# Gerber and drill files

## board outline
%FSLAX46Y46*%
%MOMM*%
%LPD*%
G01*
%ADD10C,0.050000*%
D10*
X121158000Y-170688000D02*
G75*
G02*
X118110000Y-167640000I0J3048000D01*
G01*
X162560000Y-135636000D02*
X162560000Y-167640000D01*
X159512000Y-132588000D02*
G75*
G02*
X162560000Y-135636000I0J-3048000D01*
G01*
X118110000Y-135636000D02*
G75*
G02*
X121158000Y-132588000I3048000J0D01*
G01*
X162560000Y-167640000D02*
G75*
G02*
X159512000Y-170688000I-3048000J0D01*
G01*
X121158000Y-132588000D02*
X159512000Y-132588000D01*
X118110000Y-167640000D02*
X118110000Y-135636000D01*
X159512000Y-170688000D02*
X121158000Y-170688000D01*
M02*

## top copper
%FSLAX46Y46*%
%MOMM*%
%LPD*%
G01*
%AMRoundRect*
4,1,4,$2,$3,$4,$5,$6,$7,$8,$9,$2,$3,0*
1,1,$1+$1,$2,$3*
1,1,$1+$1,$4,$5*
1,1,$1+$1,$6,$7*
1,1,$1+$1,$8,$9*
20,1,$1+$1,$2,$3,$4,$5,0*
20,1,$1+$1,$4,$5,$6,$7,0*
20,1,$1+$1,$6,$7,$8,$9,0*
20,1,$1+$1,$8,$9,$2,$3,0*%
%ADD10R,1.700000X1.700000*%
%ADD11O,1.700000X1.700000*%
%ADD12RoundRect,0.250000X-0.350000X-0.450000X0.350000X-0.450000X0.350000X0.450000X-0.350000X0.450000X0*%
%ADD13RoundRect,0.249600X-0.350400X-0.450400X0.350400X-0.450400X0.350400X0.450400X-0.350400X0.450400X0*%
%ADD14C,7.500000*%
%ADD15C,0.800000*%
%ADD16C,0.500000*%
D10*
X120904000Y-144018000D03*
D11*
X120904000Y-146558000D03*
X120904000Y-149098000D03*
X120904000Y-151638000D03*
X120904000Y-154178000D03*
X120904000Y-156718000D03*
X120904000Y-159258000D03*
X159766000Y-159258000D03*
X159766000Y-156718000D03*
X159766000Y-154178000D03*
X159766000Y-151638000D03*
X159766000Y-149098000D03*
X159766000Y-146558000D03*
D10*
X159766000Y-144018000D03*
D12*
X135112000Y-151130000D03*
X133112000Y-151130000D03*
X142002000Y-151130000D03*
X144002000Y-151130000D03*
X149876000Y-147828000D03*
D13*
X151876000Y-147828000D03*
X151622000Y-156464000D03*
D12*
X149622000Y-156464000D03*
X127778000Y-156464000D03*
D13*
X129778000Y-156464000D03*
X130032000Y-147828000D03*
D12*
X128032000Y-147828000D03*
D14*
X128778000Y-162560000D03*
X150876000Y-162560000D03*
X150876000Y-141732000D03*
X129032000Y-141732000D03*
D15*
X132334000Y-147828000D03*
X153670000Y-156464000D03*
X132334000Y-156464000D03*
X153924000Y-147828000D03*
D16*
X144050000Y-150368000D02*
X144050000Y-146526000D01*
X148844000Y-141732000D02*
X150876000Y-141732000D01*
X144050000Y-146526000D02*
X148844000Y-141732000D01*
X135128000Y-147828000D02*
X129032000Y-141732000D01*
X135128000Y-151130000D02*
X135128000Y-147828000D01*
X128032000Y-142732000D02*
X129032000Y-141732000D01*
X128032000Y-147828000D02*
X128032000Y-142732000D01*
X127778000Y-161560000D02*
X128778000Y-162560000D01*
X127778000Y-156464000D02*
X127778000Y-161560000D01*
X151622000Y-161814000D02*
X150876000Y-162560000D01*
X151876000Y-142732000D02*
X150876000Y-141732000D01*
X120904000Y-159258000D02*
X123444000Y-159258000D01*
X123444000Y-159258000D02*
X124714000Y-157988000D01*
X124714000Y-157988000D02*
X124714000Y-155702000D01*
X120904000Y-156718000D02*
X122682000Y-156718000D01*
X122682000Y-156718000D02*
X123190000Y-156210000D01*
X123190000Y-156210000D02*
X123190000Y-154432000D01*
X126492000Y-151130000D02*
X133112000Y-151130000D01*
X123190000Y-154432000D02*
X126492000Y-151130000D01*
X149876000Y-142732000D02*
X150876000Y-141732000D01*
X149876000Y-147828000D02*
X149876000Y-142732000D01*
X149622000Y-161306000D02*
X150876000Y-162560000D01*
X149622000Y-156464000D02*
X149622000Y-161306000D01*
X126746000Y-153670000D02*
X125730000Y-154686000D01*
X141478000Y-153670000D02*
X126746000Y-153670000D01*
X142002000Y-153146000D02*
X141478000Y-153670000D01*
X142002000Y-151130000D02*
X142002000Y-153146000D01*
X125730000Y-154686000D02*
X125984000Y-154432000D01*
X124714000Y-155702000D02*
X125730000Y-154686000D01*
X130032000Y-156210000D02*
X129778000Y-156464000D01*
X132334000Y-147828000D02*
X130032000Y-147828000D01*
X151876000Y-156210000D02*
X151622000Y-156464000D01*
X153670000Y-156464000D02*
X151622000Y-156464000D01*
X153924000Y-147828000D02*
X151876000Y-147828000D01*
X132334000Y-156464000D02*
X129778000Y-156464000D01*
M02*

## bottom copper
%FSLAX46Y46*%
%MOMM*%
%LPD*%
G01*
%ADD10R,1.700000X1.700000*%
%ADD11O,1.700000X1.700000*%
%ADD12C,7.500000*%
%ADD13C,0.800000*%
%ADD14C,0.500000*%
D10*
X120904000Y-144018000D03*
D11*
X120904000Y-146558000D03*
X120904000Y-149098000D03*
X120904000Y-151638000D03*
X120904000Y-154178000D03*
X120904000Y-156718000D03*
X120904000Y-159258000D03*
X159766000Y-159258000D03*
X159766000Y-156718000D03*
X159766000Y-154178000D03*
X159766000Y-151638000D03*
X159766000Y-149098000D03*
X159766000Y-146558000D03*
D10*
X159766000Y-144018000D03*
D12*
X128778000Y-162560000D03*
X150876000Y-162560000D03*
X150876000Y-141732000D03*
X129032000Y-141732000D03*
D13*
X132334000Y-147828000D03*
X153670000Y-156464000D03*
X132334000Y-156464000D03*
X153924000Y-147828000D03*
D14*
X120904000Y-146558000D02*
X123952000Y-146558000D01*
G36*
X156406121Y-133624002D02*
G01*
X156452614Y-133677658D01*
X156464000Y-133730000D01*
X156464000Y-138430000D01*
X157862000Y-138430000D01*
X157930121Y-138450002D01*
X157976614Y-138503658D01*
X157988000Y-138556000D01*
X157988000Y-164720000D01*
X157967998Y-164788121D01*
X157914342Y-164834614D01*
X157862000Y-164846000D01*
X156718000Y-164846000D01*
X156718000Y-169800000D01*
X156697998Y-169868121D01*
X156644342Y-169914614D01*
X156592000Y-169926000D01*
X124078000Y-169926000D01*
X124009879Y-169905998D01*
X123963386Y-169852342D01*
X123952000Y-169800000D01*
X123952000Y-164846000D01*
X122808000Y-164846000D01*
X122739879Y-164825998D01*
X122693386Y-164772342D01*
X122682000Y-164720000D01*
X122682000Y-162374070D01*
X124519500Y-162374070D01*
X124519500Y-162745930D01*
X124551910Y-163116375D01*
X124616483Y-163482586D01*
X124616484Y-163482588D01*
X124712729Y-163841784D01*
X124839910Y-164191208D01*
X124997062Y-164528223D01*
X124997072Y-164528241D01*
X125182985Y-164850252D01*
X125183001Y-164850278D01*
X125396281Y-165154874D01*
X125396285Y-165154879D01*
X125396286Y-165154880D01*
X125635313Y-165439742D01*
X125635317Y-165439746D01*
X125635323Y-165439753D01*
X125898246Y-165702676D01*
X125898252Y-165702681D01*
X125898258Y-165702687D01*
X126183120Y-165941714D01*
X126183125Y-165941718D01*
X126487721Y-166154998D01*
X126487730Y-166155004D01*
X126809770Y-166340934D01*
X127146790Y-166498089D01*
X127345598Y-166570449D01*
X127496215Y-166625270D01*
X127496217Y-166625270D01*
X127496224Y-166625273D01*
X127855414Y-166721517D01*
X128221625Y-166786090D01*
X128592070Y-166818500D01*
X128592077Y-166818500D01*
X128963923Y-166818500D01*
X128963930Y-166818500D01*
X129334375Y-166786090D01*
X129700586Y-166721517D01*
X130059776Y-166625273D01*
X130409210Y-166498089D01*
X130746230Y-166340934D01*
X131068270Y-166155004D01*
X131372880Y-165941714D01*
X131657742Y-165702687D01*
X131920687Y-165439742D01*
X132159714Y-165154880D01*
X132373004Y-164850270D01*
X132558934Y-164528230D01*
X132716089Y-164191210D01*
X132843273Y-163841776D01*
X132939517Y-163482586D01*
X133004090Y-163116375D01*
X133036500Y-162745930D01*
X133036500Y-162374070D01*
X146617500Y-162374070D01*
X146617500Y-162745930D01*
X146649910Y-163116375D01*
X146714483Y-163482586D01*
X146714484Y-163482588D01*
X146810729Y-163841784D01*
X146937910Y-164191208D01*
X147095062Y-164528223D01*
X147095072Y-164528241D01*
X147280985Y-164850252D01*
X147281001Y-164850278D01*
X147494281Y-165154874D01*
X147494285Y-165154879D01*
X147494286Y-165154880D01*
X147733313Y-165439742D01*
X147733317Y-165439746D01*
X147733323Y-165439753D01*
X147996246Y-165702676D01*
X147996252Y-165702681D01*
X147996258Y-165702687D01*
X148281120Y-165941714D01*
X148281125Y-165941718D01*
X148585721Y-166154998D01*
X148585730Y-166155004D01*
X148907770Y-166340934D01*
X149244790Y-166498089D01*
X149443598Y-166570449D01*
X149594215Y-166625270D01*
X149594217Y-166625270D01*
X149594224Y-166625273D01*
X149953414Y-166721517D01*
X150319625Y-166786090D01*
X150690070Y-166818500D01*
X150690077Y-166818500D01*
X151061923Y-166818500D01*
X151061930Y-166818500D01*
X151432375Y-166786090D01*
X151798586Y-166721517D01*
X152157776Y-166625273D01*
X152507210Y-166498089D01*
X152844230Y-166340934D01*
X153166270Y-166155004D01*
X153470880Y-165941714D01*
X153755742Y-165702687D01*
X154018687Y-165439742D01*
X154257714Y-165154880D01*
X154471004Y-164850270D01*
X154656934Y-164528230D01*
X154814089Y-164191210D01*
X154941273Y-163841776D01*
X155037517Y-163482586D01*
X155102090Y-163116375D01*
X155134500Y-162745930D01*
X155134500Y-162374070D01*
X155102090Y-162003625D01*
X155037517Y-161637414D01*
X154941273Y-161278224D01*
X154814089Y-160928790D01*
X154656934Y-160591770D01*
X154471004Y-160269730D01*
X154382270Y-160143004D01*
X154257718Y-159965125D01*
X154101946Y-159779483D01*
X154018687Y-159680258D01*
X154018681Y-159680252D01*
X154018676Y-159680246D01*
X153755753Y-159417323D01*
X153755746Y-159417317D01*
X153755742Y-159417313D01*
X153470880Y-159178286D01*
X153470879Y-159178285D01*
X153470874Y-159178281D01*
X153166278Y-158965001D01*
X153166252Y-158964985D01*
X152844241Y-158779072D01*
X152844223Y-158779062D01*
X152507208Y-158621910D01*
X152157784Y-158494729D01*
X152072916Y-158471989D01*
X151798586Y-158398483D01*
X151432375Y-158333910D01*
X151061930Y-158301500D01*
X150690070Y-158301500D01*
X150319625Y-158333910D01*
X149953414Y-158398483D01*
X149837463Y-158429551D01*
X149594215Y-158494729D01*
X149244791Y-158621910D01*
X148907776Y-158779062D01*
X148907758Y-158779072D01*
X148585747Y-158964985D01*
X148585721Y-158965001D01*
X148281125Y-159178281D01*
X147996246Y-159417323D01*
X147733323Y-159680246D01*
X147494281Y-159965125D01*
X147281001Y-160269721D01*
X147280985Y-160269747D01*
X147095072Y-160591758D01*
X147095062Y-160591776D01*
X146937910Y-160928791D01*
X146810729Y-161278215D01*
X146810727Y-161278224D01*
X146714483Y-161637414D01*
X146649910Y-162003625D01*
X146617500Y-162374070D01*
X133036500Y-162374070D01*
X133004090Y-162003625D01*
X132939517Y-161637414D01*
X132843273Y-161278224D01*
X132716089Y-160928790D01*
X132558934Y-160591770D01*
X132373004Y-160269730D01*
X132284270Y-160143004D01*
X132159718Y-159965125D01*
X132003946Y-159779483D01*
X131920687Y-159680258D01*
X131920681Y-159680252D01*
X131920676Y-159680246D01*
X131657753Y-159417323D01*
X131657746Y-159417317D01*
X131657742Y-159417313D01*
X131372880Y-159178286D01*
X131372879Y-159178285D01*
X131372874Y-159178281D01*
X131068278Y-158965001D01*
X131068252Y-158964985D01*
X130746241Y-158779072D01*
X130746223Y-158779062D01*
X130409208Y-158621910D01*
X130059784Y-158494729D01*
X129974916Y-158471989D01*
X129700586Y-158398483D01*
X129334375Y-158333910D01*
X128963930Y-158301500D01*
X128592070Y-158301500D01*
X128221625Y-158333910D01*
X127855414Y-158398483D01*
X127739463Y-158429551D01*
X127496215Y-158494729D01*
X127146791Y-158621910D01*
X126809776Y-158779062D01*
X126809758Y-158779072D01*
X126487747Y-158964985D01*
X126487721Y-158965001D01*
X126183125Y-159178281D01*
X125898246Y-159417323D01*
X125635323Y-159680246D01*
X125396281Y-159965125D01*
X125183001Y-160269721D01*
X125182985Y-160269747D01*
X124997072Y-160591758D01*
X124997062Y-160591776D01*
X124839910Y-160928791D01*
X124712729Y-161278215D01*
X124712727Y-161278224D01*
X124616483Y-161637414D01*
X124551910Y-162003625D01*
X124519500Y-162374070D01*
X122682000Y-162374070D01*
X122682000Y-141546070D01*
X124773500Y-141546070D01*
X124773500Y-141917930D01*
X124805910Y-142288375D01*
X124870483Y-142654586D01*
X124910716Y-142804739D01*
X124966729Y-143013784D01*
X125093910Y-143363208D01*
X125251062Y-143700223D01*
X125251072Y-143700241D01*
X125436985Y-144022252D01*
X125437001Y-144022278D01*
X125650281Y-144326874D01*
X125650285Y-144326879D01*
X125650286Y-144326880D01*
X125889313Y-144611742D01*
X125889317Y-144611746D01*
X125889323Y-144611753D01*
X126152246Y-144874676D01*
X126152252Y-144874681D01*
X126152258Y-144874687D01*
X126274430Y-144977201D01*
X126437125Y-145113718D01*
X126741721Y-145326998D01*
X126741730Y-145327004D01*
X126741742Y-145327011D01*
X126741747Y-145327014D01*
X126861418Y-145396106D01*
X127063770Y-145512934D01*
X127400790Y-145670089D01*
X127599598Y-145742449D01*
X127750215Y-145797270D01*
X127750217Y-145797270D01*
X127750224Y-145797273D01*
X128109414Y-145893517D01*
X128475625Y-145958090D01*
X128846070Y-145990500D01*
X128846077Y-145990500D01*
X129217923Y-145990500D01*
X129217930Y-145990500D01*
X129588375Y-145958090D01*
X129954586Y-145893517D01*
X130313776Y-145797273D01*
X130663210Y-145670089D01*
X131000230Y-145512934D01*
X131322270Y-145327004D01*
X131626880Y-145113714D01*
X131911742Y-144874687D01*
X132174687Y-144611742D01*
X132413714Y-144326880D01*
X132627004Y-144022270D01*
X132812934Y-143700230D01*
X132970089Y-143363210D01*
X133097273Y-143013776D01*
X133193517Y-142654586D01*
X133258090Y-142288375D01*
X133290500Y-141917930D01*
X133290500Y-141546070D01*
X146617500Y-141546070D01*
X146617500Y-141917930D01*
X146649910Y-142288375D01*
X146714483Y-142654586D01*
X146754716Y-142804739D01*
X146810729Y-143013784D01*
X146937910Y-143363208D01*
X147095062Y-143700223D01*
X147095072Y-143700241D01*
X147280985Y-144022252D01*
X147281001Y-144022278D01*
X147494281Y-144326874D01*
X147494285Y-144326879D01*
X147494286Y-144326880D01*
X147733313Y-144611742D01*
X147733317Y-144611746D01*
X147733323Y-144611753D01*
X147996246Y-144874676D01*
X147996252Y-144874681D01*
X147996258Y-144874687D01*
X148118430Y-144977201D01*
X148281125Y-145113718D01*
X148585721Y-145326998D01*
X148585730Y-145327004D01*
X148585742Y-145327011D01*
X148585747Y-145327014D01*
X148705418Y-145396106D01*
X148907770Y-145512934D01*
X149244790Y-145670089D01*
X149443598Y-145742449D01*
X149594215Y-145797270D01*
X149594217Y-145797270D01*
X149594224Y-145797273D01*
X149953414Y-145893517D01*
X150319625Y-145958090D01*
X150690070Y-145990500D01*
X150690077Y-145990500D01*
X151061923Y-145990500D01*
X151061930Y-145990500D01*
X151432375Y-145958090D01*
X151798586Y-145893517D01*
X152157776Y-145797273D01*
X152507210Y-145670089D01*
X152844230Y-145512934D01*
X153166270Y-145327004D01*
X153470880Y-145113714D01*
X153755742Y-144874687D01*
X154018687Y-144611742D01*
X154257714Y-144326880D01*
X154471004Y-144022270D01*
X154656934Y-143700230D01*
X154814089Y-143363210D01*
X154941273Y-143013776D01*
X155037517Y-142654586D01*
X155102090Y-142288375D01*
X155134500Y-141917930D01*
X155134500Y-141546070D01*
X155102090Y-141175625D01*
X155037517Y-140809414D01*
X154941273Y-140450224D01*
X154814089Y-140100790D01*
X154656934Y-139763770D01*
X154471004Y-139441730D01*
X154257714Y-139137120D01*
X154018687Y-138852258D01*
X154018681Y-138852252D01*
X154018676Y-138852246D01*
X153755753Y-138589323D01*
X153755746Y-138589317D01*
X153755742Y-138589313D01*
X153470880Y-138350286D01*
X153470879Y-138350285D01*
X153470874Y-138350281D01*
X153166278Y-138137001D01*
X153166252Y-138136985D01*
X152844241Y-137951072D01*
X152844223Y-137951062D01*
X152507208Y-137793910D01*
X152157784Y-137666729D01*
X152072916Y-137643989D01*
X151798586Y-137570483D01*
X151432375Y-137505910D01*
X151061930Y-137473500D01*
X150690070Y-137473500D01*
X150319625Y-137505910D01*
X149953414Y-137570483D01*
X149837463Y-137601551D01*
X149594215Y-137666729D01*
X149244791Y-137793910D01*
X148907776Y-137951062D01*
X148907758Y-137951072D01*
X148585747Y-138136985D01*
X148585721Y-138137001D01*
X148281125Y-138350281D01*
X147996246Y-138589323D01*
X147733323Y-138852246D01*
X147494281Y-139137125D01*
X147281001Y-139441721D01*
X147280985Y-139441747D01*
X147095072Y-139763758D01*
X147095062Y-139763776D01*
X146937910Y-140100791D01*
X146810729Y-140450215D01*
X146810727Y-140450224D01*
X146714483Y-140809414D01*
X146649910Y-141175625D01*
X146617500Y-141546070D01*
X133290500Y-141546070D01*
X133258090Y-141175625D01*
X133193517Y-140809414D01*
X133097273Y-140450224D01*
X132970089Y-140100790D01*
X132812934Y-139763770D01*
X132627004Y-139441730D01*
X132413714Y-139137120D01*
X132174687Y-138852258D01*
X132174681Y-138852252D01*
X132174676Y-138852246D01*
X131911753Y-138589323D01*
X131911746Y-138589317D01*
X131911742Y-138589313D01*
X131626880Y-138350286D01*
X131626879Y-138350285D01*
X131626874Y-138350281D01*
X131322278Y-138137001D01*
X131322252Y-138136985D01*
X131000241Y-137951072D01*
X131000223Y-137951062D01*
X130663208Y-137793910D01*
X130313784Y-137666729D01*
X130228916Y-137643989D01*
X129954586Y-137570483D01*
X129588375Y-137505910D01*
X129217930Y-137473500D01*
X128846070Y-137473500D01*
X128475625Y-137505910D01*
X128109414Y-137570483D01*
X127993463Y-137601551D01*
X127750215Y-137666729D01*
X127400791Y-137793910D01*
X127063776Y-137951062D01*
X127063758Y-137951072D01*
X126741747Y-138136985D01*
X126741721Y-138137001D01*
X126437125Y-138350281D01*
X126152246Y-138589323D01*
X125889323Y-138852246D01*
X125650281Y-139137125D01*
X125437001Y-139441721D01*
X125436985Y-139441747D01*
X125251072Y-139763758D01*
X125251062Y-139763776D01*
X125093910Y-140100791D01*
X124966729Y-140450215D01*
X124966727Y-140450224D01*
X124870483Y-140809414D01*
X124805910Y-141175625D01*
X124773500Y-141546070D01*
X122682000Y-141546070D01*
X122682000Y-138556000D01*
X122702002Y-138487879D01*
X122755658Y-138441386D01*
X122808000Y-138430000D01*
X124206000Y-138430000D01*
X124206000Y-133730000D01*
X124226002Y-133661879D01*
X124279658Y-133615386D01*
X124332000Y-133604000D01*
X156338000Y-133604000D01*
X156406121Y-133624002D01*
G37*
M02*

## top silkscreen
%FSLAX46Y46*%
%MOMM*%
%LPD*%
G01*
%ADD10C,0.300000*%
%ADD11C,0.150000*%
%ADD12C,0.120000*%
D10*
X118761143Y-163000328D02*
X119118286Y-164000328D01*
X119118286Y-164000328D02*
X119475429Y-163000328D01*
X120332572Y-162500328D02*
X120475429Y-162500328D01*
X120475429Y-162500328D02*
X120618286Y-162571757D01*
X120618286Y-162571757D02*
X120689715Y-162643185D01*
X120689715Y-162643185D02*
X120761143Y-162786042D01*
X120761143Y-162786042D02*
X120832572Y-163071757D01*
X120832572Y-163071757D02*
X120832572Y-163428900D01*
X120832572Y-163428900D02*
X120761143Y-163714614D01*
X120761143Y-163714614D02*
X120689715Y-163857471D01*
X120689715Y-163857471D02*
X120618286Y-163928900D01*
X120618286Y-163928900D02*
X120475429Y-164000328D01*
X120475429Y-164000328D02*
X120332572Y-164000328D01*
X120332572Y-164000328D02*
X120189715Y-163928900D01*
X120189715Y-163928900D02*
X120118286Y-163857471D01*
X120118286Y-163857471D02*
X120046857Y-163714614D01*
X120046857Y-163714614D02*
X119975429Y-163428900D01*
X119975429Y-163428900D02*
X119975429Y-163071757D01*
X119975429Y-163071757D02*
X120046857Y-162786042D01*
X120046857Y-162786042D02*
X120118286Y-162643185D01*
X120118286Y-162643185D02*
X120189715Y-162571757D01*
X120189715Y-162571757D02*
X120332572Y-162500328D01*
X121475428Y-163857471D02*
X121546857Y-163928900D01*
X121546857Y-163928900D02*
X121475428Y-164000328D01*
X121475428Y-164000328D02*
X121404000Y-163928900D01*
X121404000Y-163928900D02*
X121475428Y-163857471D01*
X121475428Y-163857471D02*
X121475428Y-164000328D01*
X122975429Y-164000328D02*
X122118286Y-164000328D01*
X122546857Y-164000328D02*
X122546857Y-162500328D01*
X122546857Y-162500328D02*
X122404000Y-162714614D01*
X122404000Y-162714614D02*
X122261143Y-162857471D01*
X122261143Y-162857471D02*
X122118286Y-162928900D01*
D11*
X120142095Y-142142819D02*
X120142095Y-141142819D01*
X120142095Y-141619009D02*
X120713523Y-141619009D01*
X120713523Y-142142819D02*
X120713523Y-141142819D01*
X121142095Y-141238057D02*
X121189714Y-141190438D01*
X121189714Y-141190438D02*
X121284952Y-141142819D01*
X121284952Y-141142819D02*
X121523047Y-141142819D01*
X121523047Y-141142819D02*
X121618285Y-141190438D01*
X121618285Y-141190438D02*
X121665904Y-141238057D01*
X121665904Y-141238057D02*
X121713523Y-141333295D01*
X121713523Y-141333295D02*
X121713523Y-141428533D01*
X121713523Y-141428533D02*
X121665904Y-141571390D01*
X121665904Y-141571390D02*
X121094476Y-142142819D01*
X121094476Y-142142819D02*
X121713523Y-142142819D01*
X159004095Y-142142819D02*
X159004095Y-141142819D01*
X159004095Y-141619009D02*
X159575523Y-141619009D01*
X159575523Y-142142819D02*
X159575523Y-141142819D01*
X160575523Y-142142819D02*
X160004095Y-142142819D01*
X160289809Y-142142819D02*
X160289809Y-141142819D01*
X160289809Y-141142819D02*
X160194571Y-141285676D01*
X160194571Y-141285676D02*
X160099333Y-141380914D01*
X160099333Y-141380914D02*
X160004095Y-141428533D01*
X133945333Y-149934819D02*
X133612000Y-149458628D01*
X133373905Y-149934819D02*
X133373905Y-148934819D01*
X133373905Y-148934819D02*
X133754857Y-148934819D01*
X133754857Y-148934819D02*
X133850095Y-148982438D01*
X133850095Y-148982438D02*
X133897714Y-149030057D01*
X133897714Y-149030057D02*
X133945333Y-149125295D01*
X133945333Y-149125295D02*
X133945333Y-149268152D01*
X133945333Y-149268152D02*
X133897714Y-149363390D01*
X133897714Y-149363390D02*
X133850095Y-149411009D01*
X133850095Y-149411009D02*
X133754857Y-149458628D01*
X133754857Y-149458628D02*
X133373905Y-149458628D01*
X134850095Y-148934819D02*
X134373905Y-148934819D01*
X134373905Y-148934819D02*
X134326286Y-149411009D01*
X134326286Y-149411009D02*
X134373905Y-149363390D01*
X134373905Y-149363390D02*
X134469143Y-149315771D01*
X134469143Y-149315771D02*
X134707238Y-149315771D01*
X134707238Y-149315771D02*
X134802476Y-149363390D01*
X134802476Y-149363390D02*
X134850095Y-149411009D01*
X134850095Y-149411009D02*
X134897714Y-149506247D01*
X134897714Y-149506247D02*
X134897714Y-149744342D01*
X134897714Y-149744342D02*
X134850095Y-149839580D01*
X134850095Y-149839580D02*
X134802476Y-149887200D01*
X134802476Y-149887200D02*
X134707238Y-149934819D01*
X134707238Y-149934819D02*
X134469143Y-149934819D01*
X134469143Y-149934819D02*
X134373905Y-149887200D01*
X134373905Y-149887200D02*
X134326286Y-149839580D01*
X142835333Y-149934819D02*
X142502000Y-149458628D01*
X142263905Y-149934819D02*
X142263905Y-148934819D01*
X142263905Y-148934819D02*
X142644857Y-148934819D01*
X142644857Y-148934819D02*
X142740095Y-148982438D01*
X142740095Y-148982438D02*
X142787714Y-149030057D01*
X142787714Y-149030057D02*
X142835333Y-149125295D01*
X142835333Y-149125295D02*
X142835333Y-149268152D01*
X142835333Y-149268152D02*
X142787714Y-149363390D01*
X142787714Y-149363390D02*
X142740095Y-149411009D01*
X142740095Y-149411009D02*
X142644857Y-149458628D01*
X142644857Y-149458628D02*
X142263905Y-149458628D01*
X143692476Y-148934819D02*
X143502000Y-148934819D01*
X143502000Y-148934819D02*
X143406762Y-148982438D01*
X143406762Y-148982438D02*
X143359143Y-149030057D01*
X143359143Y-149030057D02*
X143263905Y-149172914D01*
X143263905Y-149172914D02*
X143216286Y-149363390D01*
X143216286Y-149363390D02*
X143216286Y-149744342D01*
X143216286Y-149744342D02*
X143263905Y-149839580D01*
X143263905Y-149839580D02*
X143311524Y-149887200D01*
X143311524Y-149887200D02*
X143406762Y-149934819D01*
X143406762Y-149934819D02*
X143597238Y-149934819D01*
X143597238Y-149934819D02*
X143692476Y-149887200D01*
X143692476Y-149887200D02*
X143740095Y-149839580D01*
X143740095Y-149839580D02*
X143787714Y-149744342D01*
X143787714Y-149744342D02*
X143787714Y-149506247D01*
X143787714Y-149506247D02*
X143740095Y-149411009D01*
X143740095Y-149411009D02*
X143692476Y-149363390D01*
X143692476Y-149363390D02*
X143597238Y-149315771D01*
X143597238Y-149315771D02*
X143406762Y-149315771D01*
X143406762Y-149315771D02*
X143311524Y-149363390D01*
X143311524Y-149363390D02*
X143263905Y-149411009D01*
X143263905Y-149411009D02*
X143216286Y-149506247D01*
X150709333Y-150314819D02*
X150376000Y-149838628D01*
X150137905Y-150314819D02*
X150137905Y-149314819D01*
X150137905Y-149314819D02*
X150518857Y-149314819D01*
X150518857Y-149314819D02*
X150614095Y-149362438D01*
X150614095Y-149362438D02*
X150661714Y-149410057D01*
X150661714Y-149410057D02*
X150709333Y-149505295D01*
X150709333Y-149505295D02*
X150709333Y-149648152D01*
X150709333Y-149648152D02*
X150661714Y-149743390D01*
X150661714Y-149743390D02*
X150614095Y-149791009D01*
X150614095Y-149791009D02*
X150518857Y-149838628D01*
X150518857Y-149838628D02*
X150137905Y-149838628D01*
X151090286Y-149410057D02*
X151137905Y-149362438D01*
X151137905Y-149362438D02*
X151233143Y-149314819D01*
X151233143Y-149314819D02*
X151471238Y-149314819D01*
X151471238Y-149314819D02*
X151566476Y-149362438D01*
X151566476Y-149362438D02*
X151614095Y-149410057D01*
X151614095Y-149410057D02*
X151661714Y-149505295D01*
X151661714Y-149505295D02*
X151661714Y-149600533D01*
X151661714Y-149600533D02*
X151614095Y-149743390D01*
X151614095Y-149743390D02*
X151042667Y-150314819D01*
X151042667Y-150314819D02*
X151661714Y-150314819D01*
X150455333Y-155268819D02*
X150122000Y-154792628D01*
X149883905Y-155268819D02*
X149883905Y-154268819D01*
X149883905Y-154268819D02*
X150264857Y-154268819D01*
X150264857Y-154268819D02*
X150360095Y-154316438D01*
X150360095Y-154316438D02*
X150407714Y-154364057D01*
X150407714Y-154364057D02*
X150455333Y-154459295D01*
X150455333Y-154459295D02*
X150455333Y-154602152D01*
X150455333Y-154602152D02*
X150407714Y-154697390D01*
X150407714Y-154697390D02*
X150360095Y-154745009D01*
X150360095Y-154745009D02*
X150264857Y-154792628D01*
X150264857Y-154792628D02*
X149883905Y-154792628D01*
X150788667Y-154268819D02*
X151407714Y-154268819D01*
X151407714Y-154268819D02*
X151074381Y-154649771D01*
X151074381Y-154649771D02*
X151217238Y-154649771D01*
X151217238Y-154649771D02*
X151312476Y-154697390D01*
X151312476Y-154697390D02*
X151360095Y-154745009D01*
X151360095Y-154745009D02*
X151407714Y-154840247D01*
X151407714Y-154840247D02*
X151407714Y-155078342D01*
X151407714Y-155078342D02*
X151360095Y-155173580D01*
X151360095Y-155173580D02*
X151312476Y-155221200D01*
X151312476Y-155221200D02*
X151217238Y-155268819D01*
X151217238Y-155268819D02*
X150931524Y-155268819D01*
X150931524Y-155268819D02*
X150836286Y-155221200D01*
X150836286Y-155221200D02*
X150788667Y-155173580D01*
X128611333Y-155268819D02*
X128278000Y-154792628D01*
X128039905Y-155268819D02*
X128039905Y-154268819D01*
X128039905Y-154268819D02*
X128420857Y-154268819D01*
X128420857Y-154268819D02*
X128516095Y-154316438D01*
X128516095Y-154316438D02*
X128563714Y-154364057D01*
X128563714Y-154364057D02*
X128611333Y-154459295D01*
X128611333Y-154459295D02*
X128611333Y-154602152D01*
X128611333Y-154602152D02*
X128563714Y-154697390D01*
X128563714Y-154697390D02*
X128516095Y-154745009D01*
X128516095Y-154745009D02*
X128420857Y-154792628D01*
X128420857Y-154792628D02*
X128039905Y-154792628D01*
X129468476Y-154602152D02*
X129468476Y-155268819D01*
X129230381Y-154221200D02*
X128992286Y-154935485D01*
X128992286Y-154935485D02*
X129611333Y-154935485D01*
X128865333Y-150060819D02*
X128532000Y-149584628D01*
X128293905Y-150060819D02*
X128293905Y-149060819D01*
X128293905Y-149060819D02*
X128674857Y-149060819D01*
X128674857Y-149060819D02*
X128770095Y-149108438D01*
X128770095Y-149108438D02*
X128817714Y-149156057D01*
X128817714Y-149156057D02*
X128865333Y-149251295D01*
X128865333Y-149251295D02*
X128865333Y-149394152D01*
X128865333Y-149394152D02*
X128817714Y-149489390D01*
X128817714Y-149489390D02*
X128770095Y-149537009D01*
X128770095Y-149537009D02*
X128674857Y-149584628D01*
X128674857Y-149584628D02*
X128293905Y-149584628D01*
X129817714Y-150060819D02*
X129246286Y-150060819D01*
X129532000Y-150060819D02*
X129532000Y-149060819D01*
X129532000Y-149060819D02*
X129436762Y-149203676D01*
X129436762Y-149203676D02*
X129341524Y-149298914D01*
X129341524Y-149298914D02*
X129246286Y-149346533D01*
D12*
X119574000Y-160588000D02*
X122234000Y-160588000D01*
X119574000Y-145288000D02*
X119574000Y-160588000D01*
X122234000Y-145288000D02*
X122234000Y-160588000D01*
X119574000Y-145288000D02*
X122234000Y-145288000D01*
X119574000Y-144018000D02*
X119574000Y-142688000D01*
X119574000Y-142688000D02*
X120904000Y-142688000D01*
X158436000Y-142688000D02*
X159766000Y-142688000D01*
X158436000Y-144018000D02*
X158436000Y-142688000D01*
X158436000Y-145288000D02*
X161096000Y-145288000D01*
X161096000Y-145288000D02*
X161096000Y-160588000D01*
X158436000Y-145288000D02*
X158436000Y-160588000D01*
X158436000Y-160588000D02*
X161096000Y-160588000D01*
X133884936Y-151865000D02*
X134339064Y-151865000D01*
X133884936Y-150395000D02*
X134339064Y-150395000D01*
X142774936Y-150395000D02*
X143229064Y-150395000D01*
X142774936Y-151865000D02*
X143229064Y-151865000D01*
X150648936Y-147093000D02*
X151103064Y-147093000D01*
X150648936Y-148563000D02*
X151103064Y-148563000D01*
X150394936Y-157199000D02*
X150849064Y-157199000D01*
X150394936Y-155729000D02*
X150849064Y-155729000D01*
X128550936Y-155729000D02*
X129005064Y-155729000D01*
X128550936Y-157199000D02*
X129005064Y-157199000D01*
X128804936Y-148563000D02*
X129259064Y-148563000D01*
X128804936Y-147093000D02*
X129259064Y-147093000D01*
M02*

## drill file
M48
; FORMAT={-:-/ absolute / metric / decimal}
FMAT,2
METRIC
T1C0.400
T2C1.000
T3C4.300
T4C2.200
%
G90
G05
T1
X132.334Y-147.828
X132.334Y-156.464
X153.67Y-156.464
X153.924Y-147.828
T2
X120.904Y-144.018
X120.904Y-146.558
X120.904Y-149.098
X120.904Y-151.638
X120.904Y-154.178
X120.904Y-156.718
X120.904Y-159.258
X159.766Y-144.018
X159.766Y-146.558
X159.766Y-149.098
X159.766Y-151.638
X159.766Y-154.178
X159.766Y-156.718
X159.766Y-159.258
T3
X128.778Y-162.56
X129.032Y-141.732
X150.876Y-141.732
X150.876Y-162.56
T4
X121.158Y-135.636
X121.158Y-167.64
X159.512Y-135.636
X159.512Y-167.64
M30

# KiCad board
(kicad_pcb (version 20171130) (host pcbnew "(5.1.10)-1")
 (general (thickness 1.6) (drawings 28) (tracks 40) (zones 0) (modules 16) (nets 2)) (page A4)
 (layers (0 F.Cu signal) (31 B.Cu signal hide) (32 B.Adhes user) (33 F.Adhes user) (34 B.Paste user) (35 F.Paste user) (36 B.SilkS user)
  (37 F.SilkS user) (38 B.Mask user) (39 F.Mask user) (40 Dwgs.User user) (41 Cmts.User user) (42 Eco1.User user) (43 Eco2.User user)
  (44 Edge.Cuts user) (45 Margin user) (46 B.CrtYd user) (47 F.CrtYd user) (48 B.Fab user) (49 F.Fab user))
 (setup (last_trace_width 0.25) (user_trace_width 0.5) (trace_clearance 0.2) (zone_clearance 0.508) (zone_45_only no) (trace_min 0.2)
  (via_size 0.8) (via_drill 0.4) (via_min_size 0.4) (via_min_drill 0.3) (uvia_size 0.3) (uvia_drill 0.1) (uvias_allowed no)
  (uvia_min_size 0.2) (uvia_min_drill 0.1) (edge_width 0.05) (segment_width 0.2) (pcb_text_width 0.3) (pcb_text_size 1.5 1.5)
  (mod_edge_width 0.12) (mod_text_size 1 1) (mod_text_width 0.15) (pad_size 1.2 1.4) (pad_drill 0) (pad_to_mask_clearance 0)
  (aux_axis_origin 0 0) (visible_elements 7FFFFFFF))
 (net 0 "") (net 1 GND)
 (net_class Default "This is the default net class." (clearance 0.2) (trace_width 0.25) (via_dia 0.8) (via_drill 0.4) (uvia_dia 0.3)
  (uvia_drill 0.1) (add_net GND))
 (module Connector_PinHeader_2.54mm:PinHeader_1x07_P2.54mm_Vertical (layer F.Cu) (at 120.904 144.018)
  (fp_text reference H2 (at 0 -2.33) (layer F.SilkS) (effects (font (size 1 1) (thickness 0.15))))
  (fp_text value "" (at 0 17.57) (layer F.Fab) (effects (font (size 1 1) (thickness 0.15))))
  (fp_line (start -1.33 16.57) (end 1.33 16.57) (layer F.SilkS) (width 0.12))
  (fp_line (start -1.33 1.27) (end -1.33 16.57) (layer F.SilkS) (width 0.12))
  (fp_line (start 1.33 1.27) (end 1.33 16.57) (layer F.SilkS) (width 0.12))
  (fp_line (start -1.33 1.27) (end 1.33 1.27) (layer F.SilkS) (width 0.12))
  (fp_line (start -1.33 0) (end -1.33 -1.33) (layer F.SilkS) (width 0.12))
  (fp_line (start -1.33 -1.33) (end 0 -1.33) (layer F.SilkS) (width 0.12))
  (pad 1 thru_hole rect (at 0 0) (size 1.7 1.7) (drill 1) (layers *.Cu *.Mask))
  (pad 2 thru_hole oval (at 0 2.54) (size 1.7 1.7) (drill 1) (layers *.Cu *.Mask) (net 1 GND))
  (pad 3 thru_hole oval (at 0 5.08) (size 1.7 1.7) (drill 1) (layers *.Cu *.Mask))
  (pad 4 thru_hole oval (at 0 7.62) (size 1.7 1.7) (drill 1) (layers *.Cu *.Mask))
  (pad 5 thru_hole oval (at 0 10.16) (size 1.7 1.7) (drill 1) (layers *.Cu *.Mask))
  (pad 6 thru_hole oval (at 0 12.7) (size 1.7 1.7) (drill 1) (layers *.Cu *.Mask))
  (pad 7 thru_hole oval (at 0 15.24) (size 1.7 1.7) (drill 1) (layers *.Cu *.Mask)))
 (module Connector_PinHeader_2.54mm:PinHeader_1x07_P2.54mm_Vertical (layer F.Cu) (at 159.766 144.018)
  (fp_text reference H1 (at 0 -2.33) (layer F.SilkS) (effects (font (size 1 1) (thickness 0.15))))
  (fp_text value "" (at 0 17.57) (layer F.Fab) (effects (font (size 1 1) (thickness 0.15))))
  (fp_line (start -1.33 -1.33) (end 0 -1.33) (layer F.SilkS) (width 0.12))
  (fp_line (start -1.33 0) (end -1.33 -1.33) (layer F.SilkS) (width 0.12))
  (fp_line (start -1.33 1.27) (end 1.33 1.27) (layer F.SilkS) (width 0.12))
  (fp_line (start 1.33 1.27) (end 1.33 16.57) (layer F.SilkS) (width 0.12))
  (fp_line (start -1.33 1.27) (end -1.33 16.57) (layer F.SilkS) (width 0.12))
  (fp_line (start -1.33 16.57) (end 1.33 16.57) (layer F.SilkS) (width 0.12))
  (pad 7 thru_hole oval (at 0 15.24) (size 1.7 1.7) (drill 1) (layers *.Cu *.Mask))
  (pad 6 thru_hole oval (at 0 12.7) (size 1.7 1.7) (drill 1) (layers *.Cu *.Mask))
  (pad 5 thru_hole oval (at 0 10.16) (size 1.7 1.7) (drill 1) (layers *.Cu *.Mask))
  (pad 4 thru_hole oval (at 0 7.62) (size 1.7 1.7) (drill 1) (layers *.Cu *.Mask))
  (pad 3 thru_hole oval (at 0 5.08) (size 1.7 1.7) (drill 1) (layers *.Cu *.Mask))
  (pad 2 thru_hole oval (at 0 2.54) (size 1.7 1.7) (drill 1) (layers *.Cu *.Mask))
  (pad 1 thru_hole rect (at 0 0) (size 1.7 1.7) (drill 1) (layers *.Cu *.Mask)))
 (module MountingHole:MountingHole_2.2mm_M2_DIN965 (layer F.Cu) (at 159.512 167.64)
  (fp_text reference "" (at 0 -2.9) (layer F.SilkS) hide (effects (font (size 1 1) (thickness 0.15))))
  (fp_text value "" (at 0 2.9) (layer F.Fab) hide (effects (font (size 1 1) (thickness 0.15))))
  (pad 1 np_thru_hole circle (at 0 0) (size 2.2 2.2) (drill 2.2) (layers *.Cu *.Mask)))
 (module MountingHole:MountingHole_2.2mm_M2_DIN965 (layer F.Cu) (at 159.512 135.636)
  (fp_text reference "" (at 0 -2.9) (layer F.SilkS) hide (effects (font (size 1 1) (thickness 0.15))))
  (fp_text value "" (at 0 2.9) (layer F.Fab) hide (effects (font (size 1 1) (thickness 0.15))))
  (pad 1 np_thru_hole circle (at 0 0) (size 2.2 2.2) (drill 2.2) (layers *.Cu *.Mask)))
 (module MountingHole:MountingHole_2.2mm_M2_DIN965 (layer F.Cu) (at 121.158 135.636)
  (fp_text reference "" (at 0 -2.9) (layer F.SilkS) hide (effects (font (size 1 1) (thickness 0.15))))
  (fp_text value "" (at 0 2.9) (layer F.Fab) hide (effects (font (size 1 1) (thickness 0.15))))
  (pad 1 np_thru_hole circle (at 0 0) (size 2.2 2.2) (drill 2.2) (layers *.Cu *.Mask)))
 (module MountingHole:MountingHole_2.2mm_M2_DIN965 (layer F.Cu) (at 121.158 167.64)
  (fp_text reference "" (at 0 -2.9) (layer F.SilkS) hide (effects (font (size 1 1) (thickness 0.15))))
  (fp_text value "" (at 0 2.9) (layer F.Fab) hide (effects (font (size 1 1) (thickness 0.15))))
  (pad 1 np_thru_hole circle (at 0 0) (size 2.2 2.2) (drill 2.2) (layers *.Cu *.Mask)))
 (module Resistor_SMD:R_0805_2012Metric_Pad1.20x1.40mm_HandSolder (layer F.Cu) (at 134.112 151.13)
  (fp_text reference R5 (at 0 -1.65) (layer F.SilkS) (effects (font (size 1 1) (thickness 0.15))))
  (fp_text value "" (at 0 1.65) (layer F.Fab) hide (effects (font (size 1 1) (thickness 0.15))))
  (fp_line (start -0.227064 0.735) (end 0.227064 0.735) (layer F.SilkS) (width 0.12))
  (fp_line (start -0.227064 -0.735) (end 0.227064 -0.735) (layer F.SilkS) (width 0.12))
  (pad 2 smd roundrect (at 1 0) (size 1.2 1.4) (layers F.Cu F.Paste F.Mask) (roundrect_rratio 0.208333))
  (pad 1 smd roundrect (at -1 0) (size 1.2 1.4) (layers F.Cu F.Paste F.Mask) (roundrect_rratio 0.208333)))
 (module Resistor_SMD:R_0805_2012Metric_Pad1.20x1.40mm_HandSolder (layer F.Cu) (at 143.002 151.13)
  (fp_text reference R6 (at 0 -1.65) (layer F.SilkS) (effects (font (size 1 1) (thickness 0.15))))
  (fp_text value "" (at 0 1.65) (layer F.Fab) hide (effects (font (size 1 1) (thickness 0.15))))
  (fp_line (start -0.227064 -0.735) (end 0.227064 -0.735) (layer F.SilkS) (width 0.12))
  (fp_line (start -0.227064 0.735) (end 0.227064 0.735) (layer F.SilkS) (width 0.12))
  (pad 1 smd roundrect (at -1 0) (size 1.2 1.4) (layers F.Cu F.Paste F.Mask) (roundrect_rratio 0.208333))
  (pad 2 smd roundrect (at 1 0) (size 1.2 1.4) (layers F.Cu F.Paste F.Mask) (roundrect_rratio 0.208333)))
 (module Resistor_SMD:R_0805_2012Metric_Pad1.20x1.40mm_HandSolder (layer F.Cu) (at 150.876 147.828)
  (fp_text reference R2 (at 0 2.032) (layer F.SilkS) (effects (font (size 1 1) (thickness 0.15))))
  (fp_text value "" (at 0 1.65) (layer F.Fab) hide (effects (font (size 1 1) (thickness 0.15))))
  (fp_line (start -0.227064 -0.735) (end 0.227064 -0.735) (layer F.SilkS) (width 0.12))
  (fp_line (start -0.227064 0.735) (end 0.227064 0.735) (layer F.SilkS) (width 0.12))
  (pad 1 smd roundrect (at -1 0) (size 1.2 1.4) (layers F.Cu F.Paste F.Mask) (roundrect_rratio 0.208333))
  (pad 2 smd roundrect (at 1 0) (size 1.2 1.4) (layers F.Cu F.Paste F.Mask) (roundrect_rratio 0.208) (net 1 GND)))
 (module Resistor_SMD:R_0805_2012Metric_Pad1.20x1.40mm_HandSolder (layer F.Cu) (at 150.622 156.464)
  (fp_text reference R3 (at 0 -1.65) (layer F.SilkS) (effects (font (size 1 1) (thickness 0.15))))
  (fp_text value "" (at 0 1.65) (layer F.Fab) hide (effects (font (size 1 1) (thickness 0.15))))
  (fp_line (start -0.227064 0.735) (end 0.227064 0.735) (layer F.SilkS) (width 0.12))
  (fp_line (start -0.227064 -0.735) (end 0.227064 -0.735) (layer F.SilkS) (width 0.12))
  (pad 2 smd roundrect (at 1 0) (size 1.2 1.4) (layers F.Cu F.Paste F.Mask) (roundrect_rratio 0.208) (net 1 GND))
  (pad 1 smd roundrect (at -1 0) (size 1.2 1.4) (layers F.Cu F.Paste F.Mask) (roundrect_rratio 0.208333)))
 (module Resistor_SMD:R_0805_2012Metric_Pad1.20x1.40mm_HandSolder (layer F.Cu) (at 128.778 156.464)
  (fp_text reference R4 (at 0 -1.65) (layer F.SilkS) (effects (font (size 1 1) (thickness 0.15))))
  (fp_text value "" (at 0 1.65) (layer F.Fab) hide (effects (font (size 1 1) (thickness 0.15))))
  (fp_line (start -0.227064 -0.735) (end 0.227064 -0.735) (layer F.SilkS) (width 0.12))
  (fp_line (start -0.227064 0.735) (end 0.227064 0.735) (layer F.SilkS) (width 0.12))
  (pad 1 smd roundrect (at -1 0) (size 1.2 1.4) (layers F.Cu F.Paste F.Mask) (roundrect_rratio 0.208333))
  (pad 2 smd roundrect (at 1 0) (size 1.2 1.4) (layers F.Cu F.Paste F.Mask) (roundrect_rratio 0.208) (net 1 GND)))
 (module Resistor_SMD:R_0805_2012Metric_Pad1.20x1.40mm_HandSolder (layer F.Cu) (at 129.032 147.828)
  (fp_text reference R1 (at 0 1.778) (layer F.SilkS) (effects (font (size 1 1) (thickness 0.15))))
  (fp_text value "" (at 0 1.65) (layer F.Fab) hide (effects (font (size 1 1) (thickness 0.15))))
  (fp_line (start -0.227064 0.735) (end 0.227064 0.735) (layer F.SilkS) (width 0.12))
  (fp_line (start -0.227064 -0.735) (end 0.227064 -0.735) (layer F.SilkS) (width 0.12))
  (pad 2 smd roundrect (at 1 0) (size 1.2 1.4) (layers F.Cu F.Paste F.Mask) (roundrect_rratio 0.208) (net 1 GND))
  (pad 1 smd roundrect (at -1 0) (size 1.2 1.4) (layers F.Cu F.Paste F.Mask) (roundrect_rratio 0.208333)))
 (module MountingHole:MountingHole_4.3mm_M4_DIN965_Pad (layer F.Cu) (at 128.778 162.56)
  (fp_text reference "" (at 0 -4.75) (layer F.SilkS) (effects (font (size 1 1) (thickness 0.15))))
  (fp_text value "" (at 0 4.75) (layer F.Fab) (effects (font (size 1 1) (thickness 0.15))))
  (pad 1 thru_hole circle (at 0 0) (size 7.5 7.5) (drill 4.3) (layers *.Cu *.Mask)))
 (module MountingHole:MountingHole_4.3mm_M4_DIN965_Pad (layer F.Cu) (at 150.876 162.56)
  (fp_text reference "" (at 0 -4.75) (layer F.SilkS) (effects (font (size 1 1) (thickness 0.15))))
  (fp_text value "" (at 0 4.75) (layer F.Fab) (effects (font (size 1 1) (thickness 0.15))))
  (pad 1 thru_hole circle (at 0 0) (size 7.5 7.5) (drill 4.3) (layers *.Cu *.Mask)))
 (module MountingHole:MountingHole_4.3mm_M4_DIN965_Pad (layer F.Cu) (at 150.876 141.732)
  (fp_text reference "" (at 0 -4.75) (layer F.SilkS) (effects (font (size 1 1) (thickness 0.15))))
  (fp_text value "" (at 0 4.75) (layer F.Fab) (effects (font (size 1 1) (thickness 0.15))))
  (pad 1 thru_hole circle (at 0 0) (size 7.5 7.5) (drill 4.3) (layers *.Cu *.Mask)))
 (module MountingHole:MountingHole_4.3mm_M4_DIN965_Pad (layer F.Cu) (at 129.032 141.732)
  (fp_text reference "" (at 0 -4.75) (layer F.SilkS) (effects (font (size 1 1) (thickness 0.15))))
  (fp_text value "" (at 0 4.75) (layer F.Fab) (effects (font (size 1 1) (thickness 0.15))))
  (pad 1 thru_hole circle (at 0 0) (size 7.5 7.5) (drill 4.3) (layers *.Cu *.Mask)))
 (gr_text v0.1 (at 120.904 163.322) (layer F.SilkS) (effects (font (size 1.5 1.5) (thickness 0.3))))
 (gr_arc (start 121.158 167.64) (end 118.11 167.64) (angle -90) (layer Edge.Cuts) (width 0.05))
 (gr_line (start 162.56 135.636) (end 162.56 167.64) (layer Edge.Cuts) (width 0.05))
 (gr_arc (start 159.512 135.636) (end 162.56 135.636) (angle -90) (layer Edge.Cuts) (width 0.05))
 (gr_arc (start 121.158 135.636) (end 121.158 132.588) (angle -90) (layer Edge.Cuts) (width 0.05))
 (gr_arc (start 159.512 167.64) (end 159.512 170.688) (angle -90) (layer Edge.Cuts) (width 0.05))
 (gr_line (start 121.158 132.588) (end 159.512 132.588) (layer Edge.Cuts) (width 0.05))
 (gr_line (start 118.11 167.64) (end 118.11 135.636) (layer Edge.Cuts) (width 0.05))
 (gr_line (start 159.512 170.688) (end 121.158 170.688) (layer Edge.Cuts) (width 0.05))
 (segment (start 144.05 150.368) (end 144.05 146.526) (width 0.5) (layer F.Cu) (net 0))
 (segment (start 148.844 141.732) (end 150.876 141.732) (width 0.5) (layer F.Cu) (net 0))
 (segment (start 144.05 146.526) (end 148.844 141.732) (width 0.5) (layer F.Cu) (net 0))
 (segment (start 135.128 147.828) (end 129.032 141.732) (width 0.5) (layer F.Cu) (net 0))
 (segment (start 135.128 151.13) (end 135.128 147.828) (width 0.5) (layer F.Cu) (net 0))
 (segment (start 128.032 142.732) (end 129.032 141.732) (width 0.5) (layer F.Cu) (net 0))
 (segment (start 128.032 147.828) (end 128.032 142.732) (width 0.5) (layer F.Cu) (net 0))
 (segment (start 127.778 161.56) (end 128.778 162.56) (width 0.5) (layer F.Cu) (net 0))
 (segment (start 127.778 156.464) (end 127.778 161.56) (width 0.5) (layer F.Cu) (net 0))
 (segment (start 151.622 161.814) (end 150.876 162.56) (width 0.5) (layer F.Cu) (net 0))
 (segment (start 151.876 142.732) (end 150.876 141.732) (width 0.5) (layer F.Cu) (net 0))
 (segment (start 120.904 159.258) (end 123.444 159.258) (width 0.5) (layer F.Cu) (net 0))
 (segment (start 123.444 159.258) (end 124.714 157.988) (width 0.5) (layer F.Cu) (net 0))
 (segment (start 124.714 157.988) (end 124.714 155.702) (width 0.5) (layer F.Cu) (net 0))
 (segment (start 120.904 156.718) (end 122.682 156.718) (width 0.5) (layer F.Cu) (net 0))
 (segment (start 122.682 156.718) (end 123.19 156.21) (width 0.5) (layer F.Cu) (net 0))
 (segment (start 123.19 156.21) (end 123.19 154.432) (width 0.5) (layer F.Cu) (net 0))
 (segment (start 126.492 151.13) (end 133.112 151.13) (width 0.5) (layer F.Cu) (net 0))
 (segment (start 123.19 154.432) (end 126.492 151.13) (width 0.5) (layer F.Cu) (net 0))
 (segment (start 149.876 142.732) (end 150.876 141.732) (width 0.5) (layer F.Cu) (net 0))
 (segment (start 149.876 147.828) (end 149.876 142.732) (width 0.5) (layer F.Cu) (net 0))
 (segment (start 149.622 161.306) (end 150.876 162.56) (width 0.5) (layer F.Cu) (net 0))
 (segment (start 149.622 156.464) (end 149.622 161.306) (width 0.5) (layer F.Cu) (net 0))
 (segment (start 126.746 153.67) (end 125.73 154.686) (width 0.5) (layer F.Cu) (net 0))
 (segment (start 141.478 153.67) (end 126.746 153.67) (width 0.5) (layer F.Cu) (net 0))
 (segment (start 142.002 153.146) (end 141.478 153.67) (width 0.5) (layer F.Cu) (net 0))
 (segment (start 142.002 151.13) (end 142.002 153.146) (width 0.5) (layer F.Cu) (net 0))
 (segment (start 125.73 154.686) (end 125.984 154.432) (width 0.5) (layer F.Cu) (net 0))
 (segment (start 124.714 155.702) (end 125.73 154.686) (width 0.5) (layer F.Cu) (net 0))
 (segment (start 130.032 156.21) (end 129.778 156.464) (width 0.5) (layer F.Cu) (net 1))
 (via (at 132.334 147.828) (size 0.8) (drill 0.4) (layers F.Cu B.Cu) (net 1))
 (segment (start 132.334 147.828) (end 130.032 147.828) (width 0.5) (layer F.Cu) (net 1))
 (segment (start 151.876 156.21) (end 151.622 156.464) (width 0.5) (layer F.Cu) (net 1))
 (via (at 153.67 156.464) (size 0.8) (drill 0.4) (layers F.Cu B.Cu) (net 1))
 (via (at 132.334 156.464) (size 0.8) (drill 0.4) (layers F.Cu B.Cu) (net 1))
 (segment (start 153.67 156.464) (end 151.622 156.464) (width 0.5) (layer F.Cu) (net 1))
 (via (at 153.924 147.828) (size 0.8) (drill 0.4) (layers F.Cu B.Cu) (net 1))
 (segment (start 153.924 147.828) (end 151.876 147.828) (width 0.5) (layer F.Cu) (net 1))
 (segment (start 132.334 156.464) (end 129.778 156.464) (width 0.5) (layer F.Cu) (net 1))
 (segment (start 120.904 146.558) (end 123.952 146.558) (width 0.5) (layer B.Cu) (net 1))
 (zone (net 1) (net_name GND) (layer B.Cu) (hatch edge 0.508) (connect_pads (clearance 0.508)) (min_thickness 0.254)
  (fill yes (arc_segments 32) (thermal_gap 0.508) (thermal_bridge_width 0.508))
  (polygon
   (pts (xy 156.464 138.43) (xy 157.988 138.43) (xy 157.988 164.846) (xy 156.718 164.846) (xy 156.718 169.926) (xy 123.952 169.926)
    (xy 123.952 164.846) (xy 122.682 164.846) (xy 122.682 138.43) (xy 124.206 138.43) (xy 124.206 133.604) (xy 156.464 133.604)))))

